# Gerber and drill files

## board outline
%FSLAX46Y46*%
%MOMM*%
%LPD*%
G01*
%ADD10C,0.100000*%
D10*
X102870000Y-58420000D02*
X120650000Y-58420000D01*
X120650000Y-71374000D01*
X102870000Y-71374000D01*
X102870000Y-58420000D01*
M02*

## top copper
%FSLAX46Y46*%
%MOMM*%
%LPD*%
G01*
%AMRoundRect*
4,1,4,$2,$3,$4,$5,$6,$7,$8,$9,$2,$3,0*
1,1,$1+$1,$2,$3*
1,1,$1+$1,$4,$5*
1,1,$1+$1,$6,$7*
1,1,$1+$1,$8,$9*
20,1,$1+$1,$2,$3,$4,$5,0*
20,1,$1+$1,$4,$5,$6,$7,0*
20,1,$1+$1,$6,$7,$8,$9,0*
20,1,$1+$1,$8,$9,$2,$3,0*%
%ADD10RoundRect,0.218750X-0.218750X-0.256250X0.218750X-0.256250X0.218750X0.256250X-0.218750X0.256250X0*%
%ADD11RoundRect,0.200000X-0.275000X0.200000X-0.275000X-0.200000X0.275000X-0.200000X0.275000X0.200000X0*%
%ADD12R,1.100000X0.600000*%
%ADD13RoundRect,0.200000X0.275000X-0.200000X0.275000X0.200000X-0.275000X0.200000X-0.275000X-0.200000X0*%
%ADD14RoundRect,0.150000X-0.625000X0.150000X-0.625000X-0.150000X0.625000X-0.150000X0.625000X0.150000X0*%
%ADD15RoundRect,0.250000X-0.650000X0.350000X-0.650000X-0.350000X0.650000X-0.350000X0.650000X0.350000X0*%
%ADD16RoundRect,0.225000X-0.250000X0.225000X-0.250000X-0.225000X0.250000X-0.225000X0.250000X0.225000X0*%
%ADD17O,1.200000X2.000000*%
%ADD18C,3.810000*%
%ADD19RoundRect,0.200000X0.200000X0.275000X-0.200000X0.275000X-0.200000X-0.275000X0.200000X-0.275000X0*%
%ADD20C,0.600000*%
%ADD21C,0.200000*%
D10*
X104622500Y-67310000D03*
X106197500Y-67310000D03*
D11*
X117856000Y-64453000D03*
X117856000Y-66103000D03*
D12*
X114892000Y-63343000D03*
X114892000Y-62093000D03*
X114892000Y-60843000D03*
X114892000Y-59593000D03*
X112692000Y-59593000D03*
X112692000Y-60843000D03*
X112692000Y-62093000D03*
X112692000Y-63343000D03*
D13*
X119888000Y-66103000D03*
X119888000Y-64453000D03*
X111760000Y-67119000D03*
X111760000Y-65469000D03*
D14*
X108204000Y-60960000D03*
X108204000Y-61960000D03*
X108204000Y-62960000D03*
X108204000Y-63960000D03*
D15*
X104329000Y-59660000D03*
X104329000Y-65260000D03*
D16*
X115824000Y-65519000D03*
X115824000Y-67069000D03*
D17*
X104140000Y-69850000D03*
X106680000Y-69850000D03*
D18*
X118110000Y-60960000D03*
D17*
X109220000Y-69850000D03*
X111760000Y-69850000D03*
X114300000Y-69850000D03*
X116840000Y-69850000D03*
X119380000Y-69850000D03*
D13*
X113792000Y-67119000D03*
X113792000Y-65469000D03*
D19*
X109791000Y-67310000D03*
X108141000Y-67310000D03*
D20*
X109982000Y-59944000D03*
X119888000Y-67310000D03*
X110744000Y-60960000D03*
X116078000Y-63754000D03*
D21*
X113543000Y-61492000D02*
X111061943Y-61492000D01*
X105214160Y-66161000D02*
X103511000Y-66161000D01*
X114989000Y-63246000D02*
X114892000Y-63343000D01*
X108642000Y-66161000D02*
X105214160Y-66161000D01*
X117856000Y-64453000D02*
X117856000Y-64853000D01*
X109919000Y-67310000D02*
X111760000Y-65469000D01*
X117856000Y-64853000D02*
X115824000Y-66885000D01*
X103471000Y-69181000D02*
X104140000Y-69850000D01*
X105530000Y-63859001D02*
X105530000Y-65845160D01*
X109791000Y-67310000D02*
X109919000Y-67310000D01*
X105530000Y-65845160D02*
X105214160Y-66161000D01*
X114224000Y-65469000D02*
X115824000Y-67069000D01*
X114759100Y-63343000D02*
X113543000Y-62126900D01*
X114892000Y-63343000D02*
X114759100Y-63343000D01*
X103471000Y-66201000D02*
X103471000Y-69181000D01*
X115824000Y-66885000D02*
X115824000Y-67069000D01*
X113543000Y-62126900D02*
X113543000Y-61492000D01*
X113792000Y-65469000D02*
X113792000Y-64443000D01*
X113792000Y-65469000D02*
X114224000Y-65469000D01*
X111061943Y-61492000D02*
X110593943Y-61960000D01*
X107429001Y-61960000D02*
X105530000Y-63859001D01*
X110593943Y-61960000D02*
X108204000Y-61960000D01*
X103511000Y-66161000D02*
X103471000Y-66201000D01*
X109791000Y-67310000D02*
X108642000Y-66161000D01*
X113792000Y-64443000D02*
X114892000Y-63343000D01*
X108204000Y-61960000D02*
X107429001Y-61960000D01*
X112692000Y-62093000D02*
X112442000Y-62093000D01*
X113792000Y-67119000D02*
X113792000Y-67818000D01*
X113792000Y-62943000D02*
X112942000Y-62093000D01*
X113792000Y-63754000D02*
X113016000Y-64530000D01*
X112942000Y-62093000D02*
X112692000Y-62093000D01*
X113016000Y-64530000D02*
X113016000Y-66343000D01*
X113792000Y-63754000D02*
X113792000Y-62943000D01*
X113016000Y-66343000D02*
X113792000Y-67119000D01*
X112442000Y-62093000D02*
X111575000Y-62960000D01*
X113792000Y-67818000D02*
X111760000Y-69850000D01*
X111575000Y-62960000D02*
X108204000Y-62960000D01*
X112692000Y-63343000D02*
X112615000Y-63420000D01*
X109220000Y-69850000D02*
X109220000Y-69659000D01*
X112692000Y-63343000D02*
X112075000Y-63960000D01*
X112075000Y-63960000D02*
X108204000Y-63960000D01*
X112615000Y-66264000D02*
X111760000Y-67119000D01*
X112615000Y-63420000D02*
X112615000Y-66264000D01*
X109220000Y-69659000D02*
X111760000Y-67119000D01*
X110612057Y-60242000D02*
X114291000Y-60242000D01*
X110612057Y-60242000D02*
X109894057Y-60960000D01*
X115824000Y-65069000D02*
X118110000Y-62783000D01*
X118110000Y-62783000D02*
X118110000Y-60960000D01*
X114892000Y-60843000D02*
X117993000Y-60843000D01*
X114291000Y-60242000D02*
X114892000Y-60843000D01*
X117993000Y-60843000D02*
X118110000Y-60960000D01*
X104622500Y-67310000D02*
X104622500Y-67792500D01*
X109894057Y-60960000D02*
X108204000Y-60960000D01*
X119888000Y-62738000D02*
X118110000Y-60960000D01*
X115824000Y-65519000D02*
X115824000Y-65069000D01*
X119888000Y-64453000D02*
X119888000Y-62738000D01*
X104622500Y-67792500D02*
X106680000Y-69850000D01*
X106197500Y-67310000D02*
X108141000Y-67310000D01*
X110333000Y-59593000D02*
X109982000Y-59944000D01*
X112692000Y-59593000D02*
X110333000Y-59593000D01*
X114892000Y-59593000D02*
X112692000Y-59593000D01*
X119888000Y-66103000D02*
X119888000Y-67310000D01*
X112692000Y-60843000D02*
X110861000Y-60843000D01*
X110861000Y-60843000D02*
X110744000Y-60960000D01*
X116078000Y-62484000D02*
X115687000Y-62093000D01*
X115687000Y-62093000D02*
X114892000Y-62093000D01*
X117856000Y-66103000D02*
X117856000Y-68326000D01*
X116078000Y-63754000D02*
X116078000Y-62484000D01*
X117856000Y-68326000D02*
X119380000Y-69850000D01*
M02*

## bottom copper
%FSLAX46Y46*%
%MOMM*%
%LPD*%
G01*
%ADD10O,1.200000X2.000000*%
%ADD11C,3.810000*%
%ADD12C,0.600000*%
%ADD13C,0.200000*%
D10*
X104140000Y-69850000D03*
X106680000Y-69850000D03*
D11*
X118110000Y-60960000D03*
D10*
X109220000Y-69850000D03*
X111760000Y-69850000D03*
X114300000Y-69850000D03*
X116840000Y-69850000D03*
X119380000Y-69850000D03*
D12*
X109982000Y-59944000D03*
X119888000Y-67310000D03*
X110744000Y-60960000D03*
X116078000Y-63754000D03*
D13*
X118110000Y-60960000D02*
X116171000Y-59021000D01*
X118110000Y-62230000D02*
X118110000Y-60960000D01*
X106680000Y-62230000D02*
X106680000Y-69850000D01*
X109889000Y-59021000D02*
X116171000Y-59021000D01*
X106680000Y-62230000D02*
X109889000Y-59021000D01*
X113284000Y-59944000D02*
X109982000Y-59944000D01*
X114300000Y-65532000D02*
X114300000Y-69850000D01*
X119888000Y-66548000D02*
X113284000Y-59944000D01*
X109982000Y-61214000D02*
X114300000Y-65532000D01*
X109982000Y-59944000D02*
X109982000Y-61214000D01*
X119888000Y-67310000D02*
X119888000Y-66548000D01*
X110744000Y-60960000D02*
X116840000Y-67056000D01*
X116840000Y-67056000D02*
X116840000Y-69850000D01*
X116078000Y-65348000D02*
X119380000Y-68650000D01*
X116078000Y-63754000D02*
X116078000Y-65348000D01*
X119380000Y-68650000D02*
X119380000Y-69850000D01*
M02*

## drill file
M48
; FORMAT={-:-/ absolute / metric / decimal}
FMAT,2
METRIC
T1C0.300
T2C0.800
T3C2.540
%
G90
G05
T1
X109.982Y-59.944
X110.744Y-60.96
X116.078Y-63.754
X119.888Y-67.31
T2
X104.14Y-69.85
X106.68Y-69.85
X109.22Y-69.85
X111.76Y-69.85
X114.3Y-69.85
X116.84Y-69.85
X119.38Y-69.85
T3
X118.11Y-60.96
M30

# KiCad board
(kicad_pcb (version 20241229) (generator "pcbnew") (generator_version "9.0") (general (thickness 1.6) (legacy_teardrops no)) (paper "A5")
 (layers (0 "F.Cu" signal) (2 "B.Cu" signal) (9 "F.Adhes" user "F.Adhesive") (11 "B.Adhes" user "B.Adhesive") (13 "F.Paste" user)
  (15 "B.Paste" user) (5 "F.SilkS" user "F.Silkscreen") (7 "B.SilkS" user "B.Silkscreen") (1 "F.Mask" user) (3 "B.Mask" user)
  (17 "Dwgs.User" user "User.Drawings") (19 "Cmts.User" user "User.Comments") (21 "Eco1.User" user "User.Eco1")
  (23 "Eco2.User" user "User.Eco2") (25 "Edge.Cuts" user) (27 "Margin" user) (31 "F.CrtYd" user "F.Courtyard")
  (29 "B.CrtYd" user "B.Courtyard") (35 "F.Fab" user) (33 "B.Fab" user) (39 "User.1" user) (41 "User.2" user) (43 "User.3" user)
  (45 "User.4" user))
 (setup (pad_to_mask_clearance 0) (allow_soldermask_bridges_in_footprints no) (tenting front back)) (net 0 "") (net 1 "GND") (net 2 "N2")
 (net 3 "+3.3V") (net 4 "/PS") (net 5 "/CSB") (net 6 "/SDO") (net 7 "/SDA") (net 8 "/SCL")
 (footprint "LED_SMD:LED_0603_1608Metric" (layer "F.Cu") (at 105.41 67.31)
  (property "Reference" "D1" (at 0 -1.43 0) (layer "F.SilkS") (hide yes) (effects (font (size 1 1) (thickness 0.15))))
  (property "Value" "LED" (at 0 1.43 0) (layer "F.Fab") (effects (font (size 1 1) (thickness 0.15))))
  (pad "1" smd roundrect (at -0.7875 0) (size 0.875 0.95) (layers "F.Cu" "F.Mask" "F.Paste") (roundrect_rratio 0.25) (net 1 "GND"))
  (pad "2" smd roundrect (at 0.7875 0) (size 0.875 0.95) (layers "F.Cu" "F.Mask" "F.Paste") (roundrect_rratio 0.25) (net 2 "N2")))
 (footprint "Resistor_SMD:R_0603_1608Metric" (layer "F.Cu") (at 117.856 65.278 -90)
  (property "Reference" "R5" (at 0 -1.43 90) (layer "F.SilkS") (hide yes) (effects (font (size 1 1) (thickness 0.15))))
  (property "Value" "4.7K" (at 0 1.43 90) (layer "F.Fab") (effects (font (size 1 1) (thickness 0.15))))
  (pad "1" smd roundrect (at -0.825 0 270) (size 0.8 0.95) (layers "F.Cu" "F.Mask" "F.Paste") (roundrect_rratio 0.25) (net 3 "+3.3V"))
  (pad "2" smd roundrect (at 0.825 0 270) (size 0.8 0.95) (layers "F.Cu" "F.Mask" "F.Paste") (roundrect_rratio 0.25) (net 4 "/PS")))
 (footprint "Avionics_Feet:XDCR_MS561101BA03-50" (layer "F.Cu") (at 113.792 61.468 180)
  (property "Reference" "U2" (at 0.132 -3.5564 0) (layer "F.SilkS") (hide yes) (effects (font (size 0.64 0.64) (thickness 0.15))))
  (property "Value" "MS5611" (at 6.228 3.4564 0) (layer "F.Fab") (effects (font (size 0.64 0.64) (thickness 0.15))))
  (pad "1" smd rect (at -1.1 -1.875 180) (size 1.1 0.6) (layers "F.Cu" "F.Mask" "F.Paste") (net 3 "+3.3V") (solder_mask_margin 0.102))
  (pad "2" smd rect (at -1.1 -0.625 180) (size 1.1 0.6) (layers "F.Cu" "F.Mask" "F.Paste") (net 4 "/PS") (solder_mask_margin 0.102))
  (pad "3" smd rect (at -1.1 0.625 180) (size 1.1 0.6) (layers "F.Cu" "F.Mask" "F.Paste") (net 1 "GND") (solder_mask_margin 0.102))
  (pad "4" smd rect (at -1.1 1.875 180) (size 1.1 0.6) (layers "F.Cu" "F.Mask" "F.Paste") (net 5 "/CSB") (solder_mask_margin 0.102))
  (pad "5" smd rect (at 1.1 1.875 180) (size 1.1 0.6) (layers "F.Cu" "F.Mask" "F.Paste") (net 5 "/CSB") (solder_mask_margin 0.102))
  (pad "6" smd rect (at 1.1 0.625 180) (size 1.1 0.6) (layers "F.Cu" "F.Mask" "F.Paste") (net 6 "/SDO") (solder_mask_margin 0.102))
  (pad "7" smd rect (at 1.1 -0.625 180) (size 1.1 0.6) (layers "F.Cu" "F.Mask" "F.Paste") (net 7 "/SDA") (solder_mask_margin 0.102))
  (pad "8" smd rect (at 1.1 -1.875 180) (size 1.1 0.6) (layers "F.Cu" "F.Mask" "F.Paste") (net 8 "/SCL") (solder_mask_margin 0.102)))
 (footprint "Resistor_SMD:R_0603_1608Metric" (layer "F.Cu") (at 119.888 65.278 90)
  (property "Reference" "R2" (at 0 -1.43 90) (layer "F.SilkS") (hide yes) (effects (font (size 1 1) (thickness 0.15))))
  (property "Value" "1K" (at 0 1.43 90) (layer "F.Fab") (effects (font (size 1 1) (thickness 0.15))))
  (pad "1" smd roundrect (at -0.825 0 90) (size 0.8 0.95) (layers "F.Cu" "F.Mask" "F.Paste") (roundrect_rratio 0.25) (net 5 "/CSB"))
  (pad "2" smd roundrect (at 0.825 0 90) (size 0.8 0.95) (layers "F.Cu" "F.Mask" "F.Paste") (roundrect_rratio 0.25) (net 1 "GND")))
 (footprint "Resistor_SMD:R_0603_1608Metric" (layer "F.Cu") (at 111.76 66.294 90)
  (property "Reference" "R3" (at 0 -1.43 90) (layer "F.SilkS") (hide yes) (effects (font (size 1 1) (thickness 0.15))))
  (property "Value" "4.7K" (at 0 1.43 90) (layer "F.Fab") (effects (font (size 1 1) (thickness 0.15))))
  (pad "1" smd roundrect (at -0.825 0 90) (size 0.8 0.95) (layers "F.Cu" "F.Mask" "F.Paste") (roundrect_rratio 0.25) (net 8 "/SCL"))
  (pad "2" smd roundrect (at 0.825 0 90) (size 0.8 0.95) (layers "F.Cu" "F.Mask" "F.Paste") (roundrect_rratio 0.25) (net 3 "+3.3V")))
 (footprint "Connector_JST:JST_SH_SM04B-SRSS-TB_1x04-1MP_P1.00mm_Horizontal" (layer "F.Cu") (at 106.204 62.46 -90)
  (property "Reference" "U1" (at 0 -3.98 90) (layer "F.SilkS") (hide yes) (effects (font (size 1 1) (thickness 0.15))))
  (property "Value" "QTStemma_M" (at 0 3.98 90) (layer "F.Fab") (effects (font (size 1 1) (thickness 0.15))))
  (pad "1" smd roundrect (at -1.5 -2 270) (size 0.6 1.55) (layers "F.Cu" "F.Mask" "F.Paste") (roundrect_rratio 0.25) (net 1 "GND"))
  (pad "2" smd roundrect (at -0.5 -2 270) (size 0.6 1.55) (layers "F.Cu" "F.Mask" "F.Paste") (roundrect_rratio 0.25) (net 3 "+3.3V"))
  (pad "3" smd roundrect (at 0.5 -2 270) (size 0.6 1.55) (layers "F.Cu" "F.Mask" "F.Paste") (roundrect_rratio 0.25) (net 7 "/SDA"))
  (pad "4" smd roundrect (at 1.5 -2 270) (size 0.6 1.55) (layers "F.Cu" "F.Mask" "F.Paste") (roundrect_rratio 0.25) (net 8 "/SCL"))
  (pad "MP" smd roundrect (at -2.8 1.875 270) (size 1.2 1.8) (layers "F.Cu" "F.Mask" "F.Paste") (roundrect_rratio 0.208333))
  (pad "MP" smd roundrect (at 2.8 1.875 270) (size 1.2 1.8) (layers "F.Cu" "F.Mask" "F.Paste") (roundrect_rratio 0.208333)))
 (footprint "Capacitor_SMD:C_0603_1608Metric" (layer "F.Cu") (at 115.824 66.294 -90)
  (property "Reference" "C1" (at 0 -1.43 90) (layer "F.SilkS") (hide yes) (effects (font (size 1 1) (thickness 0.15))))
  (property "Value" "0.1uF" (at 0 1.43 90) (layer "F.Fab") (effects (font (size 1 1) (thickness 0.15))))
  (pad "1" smd roundrect (at -0.775 0 270) (size 0.9 0.95) (layers "F.Cu" "F.Mask" "F.Paste") (roundrect_rratio 0.25) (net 1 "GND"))
  (pad "2" smd roundrect (at 0.775 0 270) (size 0.9 0.95) (layers "F.Cu" "F.Mask" "F.Paste") (roundrect_rratio 0.25) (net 3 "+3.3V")))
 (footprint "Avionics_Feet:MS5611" (layer "F.Cu") (at 111.76 69.85)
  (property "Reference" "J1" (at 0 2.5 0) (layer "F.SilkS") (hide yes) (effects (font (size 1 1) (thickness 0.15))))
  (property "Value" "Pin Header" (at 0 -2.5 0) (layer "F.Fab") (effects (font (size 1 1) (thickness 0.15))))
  (fp_rect (start -8.89 -11.43) (end 8.89 1.524) (stroke (width 0.1) (type solid)) (fill no) (layer "Edge.Cuts"))
  (pad "1" thru_hole oval (at -7.62 0) (size 1.2 2) (drill 0.8) (layers "*.Cu" "*.Mask") (remove_unused_layers no) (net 3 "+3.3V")
   (thermal_bridge_angle 45))
  (pad "2" thru_hole oval (at -5.08 0) (size 1.2 2) (drill 0.8) (layers "*.Cu" "*.Mask") (remove_unused_layers no) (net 1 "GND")
   (thermal_bridge_angle 45))
  (pad "2" thru_hole circle (at 6.35 -8.89) (size 3.81 3.81) (drill 2.54) (layers "*.Cu" "*.Mask") (remove_unused_layers no) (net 1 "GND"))
  (pad "3" thru_hole oval (at -2.54 0) (size 1.2 2) (drill 0.8) (layers "*.Cu" "*.Mask") (remove_unused_layers no) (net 8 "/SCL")
   (thermal_bridge_angle 45))
  (pad "4" thru_hole oval (at 0 0) (size 1.2 2) (drill 0.8) (layers "*.Cu" "*.Mask") (remove_unused_layers no) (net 7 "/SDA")
   (thermal_bridge_angle 45))
  (pad "5" thru_hole oval (at 2.54 0) (size 1.2 2) (drill 0.8) (layers "*.Cu" "*.Mask") (remove_unused_layers no) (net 5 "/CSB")
   (thermal_bridge_angle 45))
  (pad "6" thru_hole oval (at 5.08 0) (size 1.2 2) (drill 0.8) (layers "*.Cu" "*.Mask") (remove_unused_layers no) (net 6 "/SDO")
   (thermal_bridge_angle 45))
  (pad "7" thru_hole oval (at 7.62 0) (size 1.2 2) (drill 0.8) (layers "*.Cu" "*.Mask") (remove_unused_layers no) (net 4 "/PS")
   (thermal_bridge_angle 45)))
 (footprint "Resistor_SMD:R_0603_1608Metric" (layer "F.Cu") (at 113.792 66.294 90)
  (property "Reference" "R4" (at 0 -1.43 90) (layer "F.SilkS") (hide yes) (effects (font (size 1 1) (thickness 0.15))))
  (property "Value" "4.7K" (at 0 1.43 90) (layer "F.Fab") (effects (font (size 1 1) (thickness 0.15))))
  (pad "1" smd roundrect (at -0.825 0 90) (size 0.8 0.95) (layers "F.Cu" "F.Mask" "F.Paste") (roundrect_rratio 0.25) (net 7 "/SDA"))
  (pad "2" smd roundrect (at 0.825 0 90) (size 0.8 0.95) (layers "F.Cu" "F.Mask" "F.Paste") (roundrect_rratio 0.25) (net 3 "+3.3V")))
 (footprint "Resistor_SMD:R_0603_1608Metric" (layer "F.Cu") (at 108.966 67.31 180)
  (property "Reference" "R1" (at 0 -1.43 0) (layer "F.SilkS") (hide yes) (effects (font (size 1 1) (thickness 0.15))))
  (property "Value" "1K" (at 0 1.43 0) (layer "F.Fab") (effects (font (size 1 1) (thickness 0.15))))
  (pad "1" smd roundrect (at -0.825 0 180) (size 0.8 0.95) (layers "F.Cu" "F.Mask" "F.Paste") (roundrect_rratio 0.25) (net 3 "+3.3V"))
  (pad "2" smd roundrect (at 0.825 0 180) (size 0.8 0.95) (layers "F.Cu" "F.Mask" "F.Paste") (roundrect_rratio 0.25) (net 2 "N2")))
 (segment (start 113.543 61.492) (end 111.061943 61.492) (width 0.2) (layer "F.Cu") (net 3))
 (segment (start 105.21416 66.161) (end 103.511 66.161) (width 0.2) (layer "F.Cu") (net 3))
 (segment (start 114.989 63.246) (end 114.892 63.343) (width 0.2) (layer "F.Cu") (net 3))
 (segment (start 108.642 66.161) (end 105.21416 66.161) (width 0.2) (layer "F.Cu") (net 3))
 (segment (start 117.856 64.453) (end 117.856 64.853) (width 0.2) (layer "F.Cu") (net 3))
 (segment (start 109.919 67.31) (end 111.76 65.469) (width 0.2) (layer "F.Cu") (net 3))
 (segment (start 117.856 64.853) (end 115.824 66.885) (width 0.2) (layer "F.Cu") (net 3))
 (segment (start 103.471 69.181) (end 104.14 69.85) (width 0.2) (layer "F.Cu") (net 3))
 (segment (start 105.53 63.859001) (end 105.53 65.84516) (width 0.2) (layer "F.Cu") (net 3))
 (segment (start 109.791 67.31) (end 109.919 67.31) (width 0.2) (layer "F.Cu") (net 3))
 (segment (start 105.53 65.84516) (end 105.21416 66.161) (width 0.2) (layer "F.Cu") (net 3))
 (segment (start 114.224 65.469) (end 115.824 67.069) (width 0.2) (layer "F.Cu") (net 3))
 (segment (start 114.7591 63.343) (end 113.543 62.1269) (width 0.2) (layer "F.Cu") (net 3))
 (segment (start 114.892 63.343) (end 114.7591 63.343) (width 0.2) (layer "F.Cu") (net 3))
 (segment (start 103.471 66.201) (end 103.471 69.181) (width 0.2) (layer "F.Cu") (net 3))
 (segment (start 115.824 66.885) (end 115.824 67.069) (width 0.2) (layer "F.Cu") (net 3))
 (segment (start 113.543 62.1269) (end 113.543 61.492) (width 0.2) (layer "F.Cu") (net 3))
 (segment (start 113.792 65.469) (end 113.792 64.443) (width 0.2) (layer "F.Cu") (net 3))
 (segment (start 113.792 65.469) (end 114.224 65.469) (width 0.2) (layer "F.Cu") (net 3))
 (segment (start 111.061943 61.492) (end 110.593943 61.96) (width 0.2) (layer "F.Cu") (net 3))
 (segment (start 107.429001 61.96) (end 105.53 63.859001) (width 0.2) (layer "F.Cu") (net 3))
 (segment (start 110.593943 61.96) (end 108.204 61.96) (width 0.2) (layer "F.Cu") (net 3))
 (segment (start 103.511 66.161) (end 103.471 66.201) (width 0.2) (layer "F.Cu") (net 3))
 (segment (start 109.791 67.31) (end 108.642 66.161) (width 0.2) (layer "F.Cu") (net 3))
 (segment (start 113.792 64.443) (end 114.892 63.343) (width 0.2) (layer "F.Cu") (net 3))
 (segment (start 108.204 61.96) (end 107.429001 61.96) (width 0.2) (layer "F.Cu") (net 3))
 (segment (start 112.692 62.093) (end 112.442 62.093) (width 0.2) (layer "F.Cu") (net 7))
 (segment (start 113.792 67.119) (end 113.792 67.818) (width 0.2) (layer "F.Cu") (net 7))
 (segment (start 113.792 62.943) (end 112.942 62.093) (width 0.2) (layer "F.Cu") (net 7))
 (segment (start 113.792 63.754) (end 113.016 64.53) (width 0.2) (layer "F.Cu") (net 7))
 (segment (start 112.942 62.093) (end 112.692 62.093) (width 0.2) (layer "F.Cu") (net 7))
 (segment (start 113.016 64.53) (end 113.016 66.343) (width 0.2) (layer "F.Cu") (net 7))
 (segment (start 113.792 63.754) (end 113.792 62.943) (width 0.2) (layer "F.Cu") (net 7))
 (segment (start 113.016 66.343) (end 113.792 67.119) (width 0.2) (layer "F.Cu") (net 7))
 (segment (start 112.442 62.093) (end 111.575 62.96) (width 0.2) (layer "F.Cu") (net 7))
 (segment (start 113.792 67.818) (end 111.76 69.85) (width 0.2) (layer "F.Cu") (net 7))
 (segment (start 111.575 62.96) (end 108.204 62.96) (width 0.2) (layer "F.Cu") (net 7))
 (segment (start 112.692 63.343) (end 112.615 63.42) (width 0.2) (layer "F.Cu") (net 8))
 (segment (start 109.22 69.85) (end 109.22 69.659) (width 0.2) (layer "F.Cu") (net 8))
 (segment (start 112.692 63.343) (end 112.075 63.96) (width 0.2) (layer "F.Cu") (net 8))
 (segment (start 112.075 63.96) (end 108.204 63.96) (width 0.2) (layer "F.Cu") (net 8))
 (segment (start 112.615 66.264) (end 111.76 67.119) (width 0.2) (layer "F.Cu") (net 8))
 (segment (start 112.615 63.42) (end 112.615 66.264) (width 0.2) (layer "F.Cu") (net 8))
 (segment (start 109.22 69.659) (end 111.76 67.119) (width 0.2) (layer "F.Cu") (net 8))
 (segment (start 110.612057 60.242) (end 114.291 60.242) (width 0.2) (layer "F.Cu") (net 1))
 (segment (start 110.612057 60.242) (end 109.894057 60.96) (width 0.2) (layer "F.Cu") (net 1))
 (segment (start 115.824 65.069) (end 118.11 62.783) (width 0.2) (layer "F.Cu") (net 1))
 (segment (start 118.11 62.783) (end 118.11 60.96) (width 0.2) (layer "F.Cu") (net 1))
 (segment (start 114.892 60.843) (end 117.993 60.843) (width 0.2) (layer "F.Cu") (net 1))
 (segment (start 114.291 60.242) (end 114.892 60.843) (width 0.2) (layer "F.Cu") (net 1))
 (segment (start 117.993 60.843) (end 118.11 60.96) (width 0.2) (layer "F.Cu") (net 1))
 (segment (start 104.6225 67.31) (end 104.6225 67.7925) (width 0.2) (layer "F.Cu") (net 1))
 (segment (start 109.894057 60.96) (end 108.204 60.96) (width 0.2) (layer "F.Cu") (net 1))
 (segment (start 119.888 62.738) (end 118.11 60.96) (width 0.2) (layer "F.Cu") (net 1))
 (segment (start 115.824 65.519) (end 115.824 65.069) (width 0.2) (layer "F.Cu") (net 1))
 (segment (start 119.888 64.453) (end 119.888 62.738) (width 0.2) (layer "F.Cu") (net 1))
 (segment (start 104.6225 67.7925) (end 106.68 69.85) (width 0.2) (layer "F.Cu") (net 1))
 (segment (start 118.11 60.96) (end 116.171 59.021) (width 0.2) (layer "B.Cu") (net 1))
 (segment (start 118.11 62.23) (end 118.11 60.96) (width 0.2) (layer "B.Cu") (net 1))
 (segment (start 106.68 62.23) (end 106.68 69.85) (width 0.2) (layer "B.Cu") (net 1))
 (segment (start 109.889 59.021) (end 116.171 59.021) (width 0.2) (layer "B.Cu") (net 1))
 (segment (start 106.68 62.23) (end 109.889 59.021) (width 0.2) (layer "B.Cu") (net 1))
 (segment (start 106.1975 67.31) (end 108.141 67.31) (width 0.2) (layer "F.Cu") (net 2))
 (segment (start 110.333 59.593) (end 109.982 59.944) (width 0.2) (layer "F.Cu") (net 5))
 (segment (start 112.692 59.593) (end 110.333 59.593) (width 0.2) (layer "F.Cu") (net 5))
 (segment (start 114.892 59.593) (end 112.692 59.593) (width 0.2) (layer "F.Cu") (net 5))
 (segment (start 119.888 66.103) (end 119.888 67.31) (width 0.2) (layer "F.Cu") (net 5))
 (via (at 109.982 59.944) (size 0.6) (drill 0.3) (layers "F.Cu" "B.Cu") (free yes) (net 5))
 (via (at 119.888 67.31) (size 0.6) (drill 0.3) (layers "F.Cu" "B.Cu") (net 5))
 (segment (start 113.284 59.944) (end 109.982 59.944) (width 0.2) (layer "B.Cu") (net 5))
 (segment (start 114.3 65.532) (end 114.3 69.85) (width 0.2) (layer "B.Cu") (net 5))
 (segment (start 119.888 66.548) (end 113.284 59.944) (width 0.2) (layer "B.Cu") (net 5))
 (segment (start 109.982 61.214) (end 114.3 65.532) (width 0.2) (layer "B.Cu") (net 5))
 (segment (start 109.982 59.944) (end 109.982 61.214) (width 0.2) (layer "B.Cu") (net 5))
 (segment (start 119.888 67.31) (end 119.888 66.548) (width 0.2) (layer "B.Cu") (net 5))
 (segment (start 112.692 60.843) (end 110.861 60.843) (width 0.2) (layer "F.Cu") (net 6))
 (segment (start 110.861 60.843) (end 110.744 60.96) (width 0.2) (layer "F.Cu") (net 6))
 (via (at 110.744 60.96) (size 0.6) (drill 0.3) (layers "F.Cu" "B.Cu") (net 6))
 (segment (start 110.744 60.96) (end 116.84 67.056) (width 0.2) (layer "B.Cu") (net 6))
 (segment (start 116.84 67.056) (end 116.84 69.85) (width 0.2) (layer "B.Cu") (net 6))
 (segment (start 116.078 62.484) (end 115.687 62.093) (width 0.2) (layer "F.Cu") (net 4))
 (segment (start 115.687 62.093) (end 114.892 62.093) (width 0.2) (layer "F.Cu") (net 4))
 (segment (start 117.856 66.103) (end 117.856 68.326) (width 0.2) (layer "F.Cu") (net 4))
 (segment (start 116.078 63.754) (end 116.078 62.484) (width 0.2) (layer "F.Cu") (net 4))
 (segment (start 117.856 68.326) (end 119.38 69.85) (width 0.2) (layer "F.Cu") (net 4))
 (via (at 116.078 63.754) (size 0.6) (drill 0.3) (layers "F.Cu" "B.Cu") (free yes) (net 4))
 (segment (start 116.078 65.348) (end 119.38 68.65) (width 0.2) (layer "B.Cu") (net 4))
 (segment (start 116.078 63.754) (end 116.078 65.348) (width 0.2) (layer "B.Cu") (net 4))
 (segment (start 119.38 68.65) (end 119.38 69.85) (width 0.2) (layer "B.Cu") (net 4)))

